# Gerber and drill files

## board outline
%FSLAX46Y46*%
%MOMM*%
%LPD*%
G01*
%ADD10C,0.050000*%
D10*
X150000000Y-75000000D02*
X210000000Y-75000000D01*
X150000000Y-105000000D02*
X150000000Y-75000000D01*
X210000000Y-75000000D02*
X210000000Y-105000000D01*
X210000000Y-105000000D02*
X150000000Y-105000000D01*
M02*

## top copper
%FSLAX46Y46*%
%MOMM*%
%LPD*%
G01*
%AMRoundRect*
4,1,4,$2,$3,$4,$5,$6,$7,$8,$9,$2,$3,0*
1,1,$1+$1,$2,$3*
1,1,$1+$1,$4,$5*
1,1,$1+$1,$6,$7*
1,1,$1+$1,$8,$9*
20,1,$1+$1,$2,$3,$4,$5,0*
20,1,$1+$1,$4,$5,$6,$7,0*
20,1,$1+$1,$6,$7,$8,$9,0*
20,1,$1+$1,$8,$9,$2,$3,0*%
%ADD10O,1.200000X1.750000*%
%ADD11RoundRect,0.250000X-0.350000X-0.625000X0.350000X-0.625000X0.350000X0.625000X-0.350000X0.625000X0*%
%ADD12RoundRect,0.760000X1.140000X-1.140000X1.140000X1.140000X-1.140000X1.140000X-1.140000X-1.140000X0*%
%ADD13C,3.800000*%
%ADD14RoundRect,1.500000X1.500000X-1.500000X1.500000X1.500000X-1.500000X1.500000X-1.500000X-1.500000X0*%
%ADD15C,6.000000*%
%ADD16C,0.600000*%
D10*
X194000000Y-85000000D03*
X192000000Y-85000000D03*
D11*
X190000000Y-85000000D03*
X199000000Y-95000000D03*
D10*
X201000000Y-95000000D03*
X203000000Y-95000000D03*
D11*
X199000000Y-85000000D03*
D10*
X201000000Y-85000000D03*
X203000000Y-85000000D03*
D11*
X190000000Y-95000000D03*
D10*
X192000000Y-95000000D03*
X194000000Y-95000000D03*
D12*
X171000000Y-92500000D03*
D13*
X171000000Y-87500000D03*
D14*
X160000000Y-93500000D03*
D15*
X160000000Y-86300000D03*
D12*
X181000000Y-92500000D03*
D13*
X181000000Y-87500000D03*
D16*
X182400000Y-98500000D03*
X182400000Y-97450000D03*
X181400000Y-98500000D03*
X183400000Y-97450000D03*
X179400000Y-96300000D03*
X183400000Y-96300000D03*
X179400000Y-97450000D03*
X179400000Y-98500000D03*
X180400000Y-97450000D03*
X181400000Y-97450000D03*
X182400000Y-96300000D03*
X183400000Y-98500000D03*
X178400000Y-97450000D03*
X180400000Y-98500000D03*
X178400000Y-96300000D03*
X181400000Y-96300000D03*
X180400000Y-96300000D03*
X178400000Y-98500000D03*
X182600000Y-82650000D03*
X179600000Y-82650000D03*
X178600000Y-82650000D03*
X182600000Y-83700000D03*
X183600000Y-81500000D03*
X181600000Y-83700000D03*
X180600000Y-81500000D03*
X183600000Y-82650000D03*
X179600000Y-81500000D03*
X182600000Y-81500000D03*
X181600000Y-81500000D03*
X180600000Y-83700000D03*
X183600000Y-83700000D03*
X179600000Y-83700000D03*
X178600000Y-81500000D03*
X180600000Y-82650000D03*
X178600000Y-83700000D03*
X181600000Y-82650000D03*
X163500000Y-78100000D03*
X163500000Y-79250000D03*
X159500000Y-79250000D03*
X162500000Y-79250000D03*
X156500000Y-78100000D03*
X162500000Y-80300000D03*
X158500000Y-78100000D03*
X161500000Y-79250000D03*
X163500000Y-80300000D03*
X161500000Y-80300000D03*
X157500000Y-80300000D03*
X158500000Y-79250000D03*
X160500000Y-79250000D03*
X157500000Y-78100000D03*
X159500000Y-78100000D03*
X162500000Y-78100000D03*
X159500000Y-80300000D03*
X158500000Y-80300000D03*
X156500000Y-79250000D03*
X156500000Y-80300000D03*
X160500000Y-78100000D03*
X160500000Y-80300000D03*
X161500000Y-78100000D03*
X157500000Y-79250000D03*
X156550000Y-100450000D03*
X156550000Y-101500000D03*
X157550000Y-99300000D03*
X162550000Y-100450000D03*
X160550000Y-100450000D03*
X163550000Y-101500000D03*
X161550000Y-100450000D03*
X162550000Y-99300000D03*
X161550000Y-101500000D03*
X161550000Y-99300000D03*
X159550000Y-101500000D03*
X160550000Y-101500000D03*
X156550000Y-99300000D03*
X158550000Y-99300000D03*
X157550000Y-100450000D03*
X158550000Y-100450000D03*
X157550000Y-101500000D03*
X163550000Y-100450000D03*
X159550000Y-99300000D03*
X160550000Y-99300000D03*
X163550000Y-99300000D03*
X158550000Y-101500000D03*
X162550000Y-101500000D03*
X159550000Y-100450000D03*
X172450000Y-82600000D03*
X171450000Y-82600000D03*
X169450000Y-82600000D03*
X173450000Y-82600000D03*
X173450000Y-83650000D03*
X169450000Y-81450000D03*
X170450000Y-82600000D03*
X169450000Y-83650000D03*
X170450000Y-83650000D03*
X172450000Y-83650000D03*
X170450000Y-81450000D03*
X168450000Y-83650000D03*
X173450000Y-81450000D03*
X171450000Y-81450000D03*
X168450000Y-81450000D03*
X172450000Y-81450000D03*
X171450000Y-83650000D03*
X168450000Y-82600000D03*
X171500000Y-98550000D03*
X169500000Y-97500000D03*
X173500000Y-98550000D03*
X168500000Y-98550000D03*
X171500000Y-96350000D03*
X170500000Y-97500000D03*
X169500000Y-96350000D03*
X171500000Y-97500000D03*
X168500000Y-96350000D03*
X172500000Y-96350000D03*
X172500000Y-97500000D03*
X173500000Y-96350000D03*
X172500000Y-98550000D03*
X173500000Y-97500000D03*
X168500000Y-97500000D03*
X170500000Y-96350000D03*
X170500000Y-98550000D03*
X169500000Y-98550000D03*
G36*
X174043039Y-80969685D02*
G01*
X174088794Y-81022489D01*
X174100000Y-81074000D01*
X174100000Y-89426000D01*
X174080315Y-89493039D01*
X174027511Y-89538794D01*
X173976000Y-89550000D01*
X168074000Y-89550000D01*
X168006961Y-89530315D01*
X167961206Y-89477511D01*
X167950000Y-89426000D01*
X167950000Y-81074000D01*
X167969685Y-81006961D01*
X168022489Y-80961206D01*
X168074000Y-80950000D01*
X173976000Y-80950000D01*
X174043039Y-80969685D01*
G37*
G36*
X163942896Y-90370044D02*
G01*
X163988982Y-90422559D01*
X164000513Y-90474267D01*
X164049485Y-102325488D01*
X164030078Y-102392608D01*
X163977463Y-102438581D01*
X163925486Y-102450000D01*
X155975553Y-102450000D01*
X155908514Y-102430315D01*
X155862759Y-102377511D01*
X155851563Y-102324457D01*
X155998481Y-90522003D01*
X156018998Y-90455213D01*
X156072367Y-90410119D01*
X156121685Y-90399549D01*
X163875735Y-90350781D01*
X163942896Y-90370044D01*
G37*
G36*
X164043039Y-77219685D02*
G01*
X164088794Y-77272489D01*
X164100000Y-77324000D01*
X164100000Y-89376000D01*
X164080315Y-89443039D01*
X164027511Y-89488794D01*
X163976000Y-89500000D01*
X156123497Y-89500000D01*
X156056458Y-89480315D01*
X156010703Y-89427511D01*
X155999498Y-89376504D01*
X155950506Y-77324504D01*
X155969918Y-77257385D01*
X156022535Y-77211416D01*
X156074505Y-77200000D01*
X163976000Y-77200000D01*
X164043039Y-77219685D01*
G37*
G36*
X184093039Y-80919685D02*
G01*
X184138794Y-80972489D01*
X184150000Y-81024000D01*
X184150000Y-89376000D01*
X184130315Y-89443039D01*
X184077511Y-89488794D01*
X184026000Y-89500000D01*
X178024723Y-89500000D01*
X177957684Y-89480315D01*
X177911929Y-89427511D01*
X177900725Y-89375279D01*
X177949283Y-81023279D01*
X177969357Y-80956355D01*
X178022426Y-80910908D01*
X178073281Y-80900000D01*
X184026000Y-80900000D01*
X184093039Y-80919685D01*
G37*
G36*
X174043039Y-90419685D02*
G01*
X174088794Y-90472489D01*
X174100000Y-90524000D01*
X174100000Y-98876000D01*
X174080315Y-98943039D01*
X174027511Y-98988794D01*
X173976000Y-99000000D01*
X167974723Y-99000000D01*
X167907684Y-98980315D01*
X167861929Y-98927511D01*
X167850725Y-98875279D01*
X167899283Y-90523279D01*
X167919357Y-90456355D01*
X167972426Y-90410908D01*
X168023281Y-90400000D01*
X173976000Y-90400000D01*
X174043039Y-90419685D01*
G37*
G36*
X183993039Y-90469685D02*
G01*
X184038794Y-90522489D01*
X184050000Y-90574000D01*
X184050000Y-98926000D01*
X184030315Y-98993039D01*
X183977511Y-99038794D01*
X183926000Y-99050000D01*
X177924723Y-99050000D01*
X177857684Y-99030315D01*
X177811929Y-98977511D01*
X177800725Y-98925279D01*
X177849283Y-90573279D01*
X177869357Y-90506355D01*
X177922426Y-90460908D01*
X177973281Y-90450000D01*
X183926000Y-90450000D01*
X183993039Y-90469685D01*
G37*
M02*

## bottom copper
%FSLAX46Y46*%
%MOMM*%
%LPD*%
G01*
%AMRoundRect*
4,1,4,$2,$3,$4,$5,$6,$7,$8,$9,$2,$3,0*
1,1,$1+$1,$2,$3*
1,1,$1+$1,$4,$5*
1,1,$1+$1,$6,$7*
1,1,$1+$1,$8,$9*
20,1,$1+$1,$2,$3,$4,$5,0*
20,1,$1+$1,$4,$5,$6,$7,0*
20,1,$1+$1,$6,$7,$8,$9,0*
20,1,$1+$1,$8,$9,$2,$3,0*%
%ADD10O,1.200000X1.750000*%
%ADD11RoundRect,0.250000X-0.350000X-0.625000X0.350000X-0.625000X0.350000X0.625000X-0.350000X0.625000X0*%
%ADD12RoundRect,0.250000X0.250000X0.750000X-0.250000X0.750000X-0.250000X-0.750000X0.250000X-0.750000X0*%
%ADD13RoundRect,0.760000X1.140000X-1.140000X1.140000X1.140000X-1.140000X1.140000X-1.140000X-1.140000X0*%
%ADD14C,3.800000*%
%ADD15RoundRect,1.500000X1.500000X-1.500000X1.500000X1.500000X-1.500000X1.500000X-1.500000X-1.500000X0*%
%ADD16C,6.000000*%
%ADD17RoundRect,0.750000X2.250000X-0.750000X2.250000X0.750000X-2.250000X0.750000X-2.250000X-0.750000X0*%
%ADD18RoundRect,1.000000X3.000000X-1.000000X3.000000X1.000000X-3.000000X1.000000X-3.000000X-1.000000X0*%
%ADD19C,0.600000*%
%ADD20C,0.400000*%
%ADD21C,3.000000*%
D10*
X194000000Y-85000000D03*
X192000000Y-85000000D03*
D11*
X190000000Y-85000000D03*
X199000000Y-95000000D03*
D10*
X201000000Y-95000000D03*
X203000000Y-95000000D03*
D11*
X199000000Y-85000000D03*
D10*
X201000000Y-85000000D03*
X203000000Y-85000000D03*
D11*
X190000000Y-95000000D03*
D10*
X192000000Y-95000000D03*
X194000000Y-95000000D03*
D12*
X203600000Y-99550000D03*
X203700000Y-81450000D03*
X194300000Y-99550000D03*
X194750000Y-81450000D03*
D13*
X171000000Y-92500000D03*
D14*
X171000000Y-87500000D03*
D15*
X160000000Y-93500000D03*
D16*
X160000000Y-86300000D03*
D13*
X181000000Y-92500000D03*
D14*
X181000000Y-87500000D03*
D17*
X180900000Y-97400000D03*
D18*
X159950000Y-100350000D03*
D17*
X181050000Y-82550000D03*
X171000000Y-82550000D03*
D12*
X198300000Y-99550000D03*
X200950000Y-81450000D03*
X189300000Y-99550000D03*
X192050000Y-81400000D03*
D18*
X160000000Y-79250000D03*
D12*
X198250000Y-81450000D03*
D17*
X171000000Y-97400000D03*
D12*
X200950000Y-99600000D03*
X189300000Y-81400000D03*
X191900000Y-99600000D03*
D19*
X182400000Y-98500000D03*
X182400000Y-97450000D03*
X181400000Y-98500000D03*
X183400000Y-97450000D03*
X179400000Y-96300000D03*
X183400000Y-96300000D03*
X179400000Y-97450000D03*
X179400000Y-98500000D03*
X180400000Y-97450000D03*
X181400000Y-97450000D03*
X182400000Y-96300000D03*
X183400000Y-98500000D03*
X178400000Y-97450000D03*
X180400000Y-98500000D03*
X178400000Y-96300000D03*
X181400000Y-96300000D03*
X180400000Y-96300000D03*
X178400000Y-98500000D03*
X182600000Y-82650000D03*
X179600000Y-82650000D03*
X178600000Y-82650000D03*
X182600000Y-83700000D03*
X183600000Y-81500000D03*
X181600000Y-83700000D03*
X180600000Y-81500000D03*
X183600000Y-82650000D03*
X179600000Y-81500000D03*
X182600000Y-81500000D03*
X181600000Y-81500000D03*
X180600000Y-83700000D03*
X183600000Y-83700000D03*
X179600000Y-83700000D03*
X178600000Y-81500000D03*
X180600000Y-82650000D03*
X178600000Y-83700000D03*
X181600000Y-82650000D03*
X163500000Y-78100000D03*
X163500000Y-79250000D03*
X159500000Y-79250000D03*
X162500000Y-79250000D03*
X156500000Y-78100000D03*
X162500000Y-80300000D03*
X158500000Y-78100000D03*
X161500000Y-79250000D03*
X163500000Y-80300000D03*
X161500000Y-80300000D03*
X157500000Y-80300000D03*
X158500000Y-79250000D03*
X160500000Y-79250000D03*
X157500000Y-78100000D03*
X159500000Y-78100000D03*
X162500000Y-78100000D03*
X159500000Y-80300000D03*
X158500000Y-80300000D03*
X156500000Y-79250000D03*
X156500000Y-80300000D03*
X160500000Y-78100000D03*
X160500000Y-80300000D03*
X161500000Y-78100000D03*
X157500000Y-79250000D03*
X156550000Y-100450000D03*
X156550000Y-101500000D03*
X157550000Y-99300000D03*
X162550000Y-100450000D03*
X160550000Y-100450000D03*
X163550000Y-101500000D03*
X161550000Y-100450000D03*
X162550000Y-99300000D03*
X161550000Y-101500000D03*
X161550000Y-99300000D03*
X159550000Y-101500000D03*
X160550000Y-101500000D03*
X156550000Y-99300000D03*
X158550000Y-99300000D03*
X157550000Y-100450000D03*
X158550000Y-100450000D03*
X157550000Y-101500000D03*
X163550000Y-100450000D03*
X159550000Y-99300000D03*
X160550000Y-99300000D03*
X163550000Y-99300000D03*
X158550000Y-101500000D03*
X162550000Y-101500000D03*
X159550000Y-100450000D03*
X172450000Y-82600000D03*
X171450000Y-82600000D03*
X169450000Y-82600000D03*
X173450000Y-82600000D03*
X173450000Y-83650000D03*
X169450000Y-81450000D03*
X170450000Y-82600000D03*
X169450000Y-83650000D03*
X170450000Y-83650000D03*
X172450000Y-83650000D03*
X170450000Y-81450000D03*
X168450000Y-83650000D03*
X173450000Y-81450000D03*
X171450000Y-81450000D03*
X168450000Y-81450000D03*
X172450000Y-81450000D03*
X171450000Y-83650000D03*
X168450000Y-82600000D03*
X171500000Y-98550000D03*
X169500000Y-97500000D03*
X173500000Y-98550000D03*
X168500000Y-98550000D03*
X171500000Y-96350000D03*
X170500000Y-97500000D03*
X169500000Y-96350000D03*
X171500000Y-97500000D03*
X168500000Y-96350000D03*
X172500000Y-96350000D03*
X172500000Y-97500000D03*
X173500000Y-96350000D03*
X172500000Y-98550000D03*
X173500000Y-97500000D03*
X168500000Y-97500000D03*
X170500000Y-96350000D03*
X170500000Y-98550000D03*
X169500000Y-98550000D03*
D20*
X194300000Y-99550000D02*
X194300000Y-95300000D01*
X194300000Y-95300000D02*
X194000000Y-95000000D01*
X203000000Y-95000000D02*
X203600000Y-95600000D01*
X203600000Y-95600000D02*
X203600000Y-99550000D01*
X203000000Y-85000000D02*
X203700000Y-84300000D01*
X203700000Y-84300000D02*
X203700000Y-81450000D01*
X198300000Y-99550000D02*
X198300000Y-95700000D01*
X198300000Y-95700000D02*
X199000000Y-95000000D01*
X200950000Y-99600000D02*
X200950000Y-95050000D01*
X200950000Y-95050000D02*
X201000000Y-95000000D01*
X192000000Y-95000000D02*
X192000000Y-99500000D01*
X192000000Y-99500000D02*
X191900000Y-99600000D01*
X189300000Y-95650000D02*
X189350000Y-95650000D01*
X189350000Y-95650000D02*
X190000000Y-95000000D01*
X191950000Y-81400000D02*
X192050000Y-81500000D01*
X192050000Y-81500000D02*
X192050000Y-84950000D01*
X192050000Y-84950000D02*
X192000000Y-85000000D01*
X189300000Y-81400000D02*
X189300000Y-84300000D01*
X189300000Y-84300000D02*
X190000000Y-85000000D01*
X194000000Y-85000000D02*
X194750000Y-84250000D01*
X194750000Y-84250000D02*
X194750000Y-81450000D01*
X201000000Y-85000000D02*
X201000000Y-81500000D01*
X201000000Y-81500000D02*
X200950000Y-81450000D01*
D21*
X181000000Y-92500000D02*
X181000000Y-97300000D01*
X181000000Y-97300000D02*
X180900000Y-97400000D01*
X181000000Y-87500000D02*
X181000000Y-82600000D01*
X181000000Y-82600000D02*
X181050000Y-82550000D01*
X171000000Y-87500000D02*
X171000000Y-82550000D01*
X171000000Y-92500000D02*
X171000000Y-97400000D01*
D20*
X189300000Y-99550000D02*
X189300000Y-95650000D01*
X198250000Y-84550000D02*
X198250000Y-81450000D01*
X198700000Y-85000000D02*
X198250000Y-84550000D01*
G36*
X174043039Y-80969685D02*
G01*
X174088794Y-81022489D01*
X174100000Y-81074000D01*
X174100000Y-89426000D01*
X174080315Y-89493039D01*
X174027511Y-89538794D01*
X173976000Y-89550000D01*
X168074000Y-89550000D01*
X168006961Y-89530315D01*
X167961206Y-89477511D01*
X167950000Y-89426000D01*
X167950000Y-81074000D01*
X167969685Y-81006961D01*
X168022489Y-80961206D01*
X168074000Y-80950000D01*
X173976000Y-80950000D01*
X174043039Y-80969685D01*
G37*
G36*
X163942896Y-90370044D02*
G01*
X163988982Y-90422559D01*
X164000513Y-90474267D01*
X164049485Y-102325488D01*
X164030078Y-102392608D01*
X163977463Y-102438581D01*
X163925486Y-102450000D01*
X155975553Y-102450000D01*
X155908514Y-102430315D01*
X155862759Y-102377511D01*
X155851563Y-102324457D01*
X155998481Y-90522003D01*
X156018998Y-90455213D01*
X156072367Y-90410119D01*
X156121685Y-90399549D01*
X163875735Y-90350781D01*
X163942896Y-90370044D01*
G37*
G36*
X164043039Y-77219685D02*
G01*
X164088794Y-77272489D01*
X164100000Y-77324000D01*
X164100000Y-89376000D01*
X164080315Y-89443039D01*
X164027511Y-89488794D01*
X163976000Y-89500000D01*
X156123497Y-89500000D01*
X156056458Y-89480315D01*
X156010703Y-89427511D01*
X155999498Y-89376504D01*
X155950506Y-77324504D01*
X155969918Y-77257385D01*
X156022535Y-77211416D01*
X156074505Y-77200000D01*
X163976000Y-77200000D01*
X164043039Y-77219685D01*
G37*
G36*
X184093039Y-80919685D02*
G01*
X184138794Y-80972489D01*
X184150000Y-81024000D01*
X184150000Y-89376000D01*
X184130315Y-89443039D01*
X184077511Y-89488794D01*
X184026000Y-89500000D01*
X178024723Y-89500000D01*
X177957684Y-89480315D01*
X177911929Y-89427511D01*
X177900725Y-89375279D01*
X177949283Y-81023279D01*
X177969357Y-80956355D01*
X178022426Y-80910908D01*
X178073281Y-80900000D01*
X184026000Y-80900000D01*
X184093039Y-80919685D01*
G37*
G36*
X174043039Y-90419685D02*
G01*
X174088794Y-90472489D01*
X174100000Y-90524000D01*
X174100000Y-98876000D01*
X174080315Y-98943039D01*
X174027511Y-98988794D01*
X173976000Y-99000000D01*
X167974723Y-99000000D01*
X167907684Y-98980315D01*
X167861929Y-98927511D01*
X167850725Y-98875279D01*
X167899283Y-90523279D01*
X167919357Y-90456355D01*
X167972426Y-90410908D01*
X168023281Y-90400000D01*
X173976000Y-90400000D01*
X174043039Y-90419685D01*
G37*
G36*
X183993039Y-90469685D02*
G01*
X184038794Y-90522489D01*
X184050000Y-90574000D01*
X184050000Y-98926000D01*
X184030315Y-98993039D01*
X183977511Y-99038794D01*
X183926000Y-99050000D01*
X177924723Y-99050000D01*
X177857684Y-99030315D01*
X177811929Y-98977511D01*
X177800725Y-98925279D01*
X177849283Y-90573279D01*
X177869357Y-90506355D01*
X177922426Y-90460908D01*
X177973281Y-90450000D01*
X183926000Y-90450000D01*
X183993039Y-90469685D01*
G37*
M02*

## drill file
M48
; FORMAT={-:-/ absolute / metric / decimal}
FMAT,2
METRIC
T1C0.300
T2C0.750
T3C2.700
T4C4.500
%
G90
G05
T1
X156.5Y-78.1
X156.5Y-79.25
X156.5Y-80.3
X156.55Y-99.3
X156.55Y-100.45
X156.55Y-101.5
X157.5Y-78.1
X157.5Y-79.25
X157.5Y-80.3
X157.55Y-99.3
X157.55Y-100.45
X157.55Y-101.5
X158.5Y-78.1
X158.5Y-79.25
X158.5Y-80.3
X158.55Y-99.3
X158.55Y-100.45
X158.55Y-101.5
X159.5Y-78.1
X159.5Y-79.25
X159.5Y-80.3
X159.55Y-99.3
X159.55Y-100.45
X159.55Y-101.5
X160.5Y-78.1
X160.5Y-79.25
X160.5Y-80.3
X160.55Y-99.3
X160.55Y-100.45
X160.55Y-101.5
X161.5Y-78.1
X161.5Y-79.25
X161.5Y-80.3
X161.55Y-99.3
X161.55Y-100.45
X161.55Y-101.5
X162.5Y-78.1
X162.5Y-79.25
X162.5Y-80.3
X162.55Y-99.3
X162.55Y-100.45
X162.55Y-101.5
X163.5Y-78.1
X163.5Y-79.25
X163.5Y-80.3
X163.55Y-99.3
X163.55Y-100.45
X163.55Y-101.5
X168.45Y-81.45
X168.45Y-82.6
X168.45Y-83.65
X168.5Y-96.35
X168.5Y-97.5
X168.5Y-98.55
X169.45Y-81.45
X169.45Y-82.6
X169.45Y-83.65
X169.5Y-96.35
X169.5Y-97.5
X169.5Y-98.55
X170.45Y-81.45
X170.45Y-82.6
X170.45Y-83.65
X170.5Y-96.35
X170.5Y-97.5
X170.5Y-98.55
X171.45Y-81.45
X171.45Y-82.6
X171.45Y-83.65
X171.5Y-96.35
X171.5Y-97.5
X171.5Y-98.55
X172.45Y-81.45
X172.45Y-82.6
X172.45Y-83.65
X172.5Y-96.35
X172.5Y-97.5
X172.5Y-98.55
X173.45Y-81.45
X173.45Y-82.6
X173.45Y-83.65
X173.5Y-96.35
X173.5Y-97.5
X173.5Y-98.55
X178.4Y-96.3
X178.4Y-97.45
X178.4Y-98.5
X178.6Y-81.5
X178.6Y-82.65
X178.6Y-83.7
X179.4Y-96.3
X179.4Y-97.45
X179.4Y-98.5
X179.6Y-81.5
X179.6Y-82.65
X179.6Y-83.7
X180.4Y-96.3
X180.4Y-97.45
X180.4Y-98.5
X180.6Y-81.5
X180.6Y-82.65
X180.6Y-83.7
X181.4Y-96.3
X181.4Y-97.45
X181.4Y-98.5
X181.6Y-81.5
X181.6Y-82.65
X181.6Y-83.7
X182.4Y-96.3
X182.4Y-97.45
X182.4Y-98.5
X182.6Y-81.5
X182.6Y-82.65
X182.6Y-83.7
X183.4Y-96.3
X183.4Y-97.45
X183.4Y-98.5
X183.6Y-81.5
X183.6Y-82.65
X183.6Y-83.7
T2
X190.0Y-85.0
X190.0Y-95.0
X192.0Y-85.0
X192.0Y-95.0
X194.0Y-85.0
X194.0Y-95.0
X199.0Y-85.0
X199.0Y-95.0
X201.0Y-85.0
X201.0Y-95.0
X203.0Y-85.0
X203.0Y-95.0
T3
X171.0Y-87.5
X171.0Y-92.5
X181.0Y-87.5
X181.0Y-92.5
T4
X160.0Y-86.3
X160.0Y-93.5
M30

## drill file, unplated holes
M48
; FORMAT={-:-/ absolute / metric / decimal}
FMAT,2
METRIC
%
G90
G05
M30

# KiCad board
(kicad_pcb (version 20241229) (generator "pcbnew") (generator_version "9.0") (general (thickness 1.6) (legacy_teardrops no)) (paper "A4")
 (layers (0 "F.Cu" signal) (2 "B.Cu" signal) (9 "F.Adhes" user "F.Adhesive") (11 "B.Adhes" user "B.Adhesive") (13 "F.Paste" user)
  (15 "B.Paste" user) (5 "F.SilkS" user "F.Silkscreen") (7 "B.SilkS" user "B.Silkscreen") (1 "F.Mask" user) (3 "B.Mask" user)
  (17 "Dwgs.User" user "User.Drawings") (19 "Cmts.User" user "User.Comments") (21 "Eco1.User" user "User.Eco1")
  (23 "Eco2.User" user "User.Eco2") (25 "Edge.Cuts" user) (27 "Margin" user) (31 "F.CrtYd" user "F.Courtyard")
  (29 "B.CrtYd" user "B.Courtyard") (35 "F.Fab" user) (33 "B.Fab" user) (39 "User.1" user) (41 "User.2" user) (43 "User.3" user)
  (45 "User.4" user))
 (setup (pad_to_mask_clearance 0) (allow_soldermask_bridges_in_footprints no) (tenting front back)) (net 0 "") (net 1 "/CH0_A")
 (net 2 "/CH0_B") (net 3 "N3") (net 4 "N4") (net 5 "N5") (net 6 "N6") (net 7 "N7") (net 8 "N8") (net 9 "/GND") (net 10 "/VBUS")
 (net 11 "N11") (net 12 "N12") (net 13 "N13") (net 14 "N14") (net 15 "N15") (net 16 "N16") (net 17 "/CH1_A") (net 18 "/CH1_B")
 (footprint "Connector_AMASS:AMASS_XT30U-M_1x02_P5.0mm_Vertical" (layer "F.Cu") (at 171 92.5 90)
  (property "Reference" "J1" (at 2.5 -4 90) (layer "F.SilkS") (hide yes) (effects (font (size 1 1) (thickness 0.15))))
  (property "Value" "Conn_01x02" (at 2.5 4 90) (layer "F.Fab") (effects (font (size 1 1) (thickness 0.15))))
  (pad "1" thru_hole roundrect (at 0 0 90) (size 3.8 3.8) (drill 2.7) (layers "*.Cu" "*.Mask") (remove_unused_layers no)
   (roundrect_rratio 0.2) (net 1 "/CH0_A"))
  (pad "2" thru_hole circle (at 5 0 90) (size 3.8 3.8) (drill 2.7) (layers "*.Cu" "*.Mask") (remove_unused_layers no) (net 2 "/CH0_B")))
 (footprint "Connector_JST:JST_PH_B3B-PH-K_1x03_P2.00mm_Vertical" (layer "F.Cu") (at 190 85)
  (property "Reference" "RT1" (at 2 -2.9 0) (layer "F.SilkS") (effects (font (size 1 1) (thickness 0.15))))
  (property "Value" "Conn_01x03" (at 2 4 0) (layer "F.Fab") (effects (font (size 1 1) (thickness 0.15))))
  (pad "1" thru_hole roundrect (at 0 0) (size 1.2 1.75) (drill 0.75) (layers "*.Cu" "*.Mask") (remove_unused_layers no)
   (roundrect_rratio 0.208333) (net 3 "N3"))
  (pad "2" thru_hole oval (at 2 0) (size 1.2 1.75) (drill 0.75) (layers "*.Cu" "*.Mask") (remove_unused_layers no) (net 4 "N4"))
  (pad "3" thru_hole oval (at 4 0) (size 1.2 1.75) (drill 0.75) (layers "*.Cu" "*.Mask") (remove_unused_layers no) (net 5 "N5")))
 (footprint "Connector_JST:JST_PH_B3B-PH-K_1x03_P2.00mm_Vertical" (layer "F.Cu") (at 199 95)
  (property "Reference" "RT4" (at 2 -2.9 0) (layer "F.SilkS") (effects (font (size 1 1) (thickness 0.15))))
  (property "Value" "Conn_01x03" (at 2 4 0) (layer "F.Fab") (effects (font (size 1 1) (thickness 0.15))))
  (pad "1" thru_hole roundrect (at 0 0) (size 1.2 1.75) (drill 0.75) (layers "*.Cu" "*.Mask") (remove_unused_layers no)
   (roundrect_rratio 0.208333) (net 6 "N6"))
  (pad "2" thru_hole oval (at 2 0) (size 1.2 1.75) (drill 0.75) (layers "*.Cu" "*.Mask") (remove_unused_layers no) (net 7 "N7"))
  (pad "3" thru_hole oval (at 4 0) (size 1.2 1.75) (drill 0.75) (layers "*.Cu" "*.Mask") (remove_unused_layers no) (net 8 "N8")))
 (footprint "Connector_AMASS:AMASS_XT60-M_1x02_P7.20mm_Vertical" (layer "F.Cu") (at 160 93.5 90)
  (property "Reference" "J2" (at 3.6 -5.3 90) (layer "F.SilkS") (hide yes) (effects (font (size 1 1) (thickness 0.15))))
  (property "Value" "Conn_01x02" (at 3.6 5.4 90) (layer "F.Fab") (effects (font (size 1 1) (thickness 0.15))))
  (pad "1" thru_hole roundrect (at 0 0 90) (size 6 6) (drill 4.5) (layers "*.Cu" "*.Mask") (remove_unused_layers no) (roundrect_rratio 0.25)
   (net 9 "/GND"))
  (pad "2" thru_hole circle (at 7.2 0 90) (size 6 6) (drill 4.5) (layers "*.Cu" "*.Mask") (remove_unused_layers no) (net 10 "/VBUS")))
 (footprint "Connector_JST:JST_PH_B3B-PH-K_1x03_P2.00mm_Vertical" (layer "F.Cu") (at 199 85)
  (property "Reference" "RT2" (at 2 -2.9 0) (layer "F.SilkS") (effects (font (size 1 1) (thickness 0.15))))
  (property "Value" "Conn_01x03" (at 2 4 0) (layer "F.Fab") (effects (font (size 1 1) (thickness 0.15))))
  (pad "1" thru_hole roundrect (at 0 0) (size 1.2 1.75) (drill 0.75) (layers "*.Cu" "*.Mask") (remove_unused_layers no)
   (roundrect_rratio 0.208333) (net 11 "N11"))
  (pad "2" thru_hole oval (at 2 0) (size 1.2 1.75) (drill 0.75) (layers "*.Cu" "*.Mask") (remove_unused_layers no) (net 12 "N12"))
  (pad "3" thru_hole oval (at 4 0) (size 1.2 1.75) (drill 0.75) (layers "*.Cu" "*.Mask") (remove_unused_layers no) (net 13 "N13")))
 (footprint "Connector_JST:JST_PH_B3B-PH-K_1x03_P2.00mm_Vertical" (layer "F.Cu") (at 190 95)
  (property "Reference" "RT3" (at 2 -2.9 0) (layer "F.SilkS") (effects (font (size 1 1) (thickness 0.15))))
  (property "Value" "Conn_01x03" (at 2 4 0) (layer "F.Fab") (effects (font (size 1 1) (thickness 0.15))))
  (pad "1" thru_hole roundrect (at 0 0) (size 1.2 1.75) (drill 0.75) (layers "*.Cu" "*.Mask") (remove_unused_layers no)
   (roundrect_rratio 0.208333) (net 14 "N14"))
  (pad "2" thru_hole oval (at 2 0) (size 1.2 1.75) (drill 0.75) (layers "*.Cu" "*.Mask") (remove_unused_layers no) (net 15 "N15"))
  (pad "3" thru_hole oval (at 4 0) (size 1.2 1.75) (drill 0.75) (layers "*.Cu" "*.Mask") (remove_unused_layers no) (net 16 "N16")))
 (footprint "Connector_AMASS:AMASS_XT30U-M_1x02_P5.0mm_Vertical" (layer "F.Cu") (at 181 92.5 90)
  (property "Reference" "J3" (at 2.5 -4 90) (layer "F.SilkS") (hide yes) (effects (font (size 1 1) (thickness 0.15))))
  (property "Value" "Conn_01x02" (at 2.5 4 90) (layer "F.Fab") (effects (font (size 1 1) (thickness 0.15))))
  (pad "1" thru_hole roundrect (at 0 0 90) (size 3.8 3.8) (drill 2.7) (layers "*.Cu" "*.Mask") (remove_unused_layers no)
   (roundrect_rratio 0.2) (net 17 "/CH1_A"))
  (pad "2" thru_hole circle (at 5 0 90) (size 3.8 3.8) (drill 2.7) (layers "*.Cu" "*.Mask") (remove_unused_layers no) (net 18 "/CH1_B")))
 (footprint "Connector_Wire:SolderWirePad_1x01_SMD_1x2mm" (layer "B.Cu") (at 203.7 81.45 180)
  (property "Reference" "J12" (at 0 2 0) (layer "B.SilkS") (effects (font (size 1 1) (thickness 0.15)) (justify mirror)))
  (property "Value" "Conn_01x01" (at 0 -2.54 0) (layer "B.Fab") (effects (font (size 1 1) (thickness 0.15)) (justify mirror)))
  (pad "1" smd roundrect (at 0 0 180) (size 1 2) (layers "B.Cu" "B.Mask") (roundrect_rratio 0.25) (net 13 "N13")))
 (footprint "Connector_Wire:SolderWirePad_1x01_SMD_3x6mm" (layer "B.Cu") (at 180.9 97.4 90)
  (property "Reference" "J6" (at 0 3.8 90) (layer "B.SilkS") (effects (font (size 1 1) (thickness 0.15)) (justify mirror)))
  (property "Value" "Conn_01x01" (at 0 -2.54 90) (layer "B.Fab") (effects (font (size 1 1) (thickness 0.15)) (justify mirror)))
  (pad "1" smd roundrect (at 0 0 90) (size 3 6) (layers "B.Cu" "B.Mask") (roundrect_rratio 0.25) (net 17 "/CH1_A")))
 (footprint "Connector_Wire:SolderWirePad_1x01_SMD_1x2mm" (layer "B.Cu") (at 203.6 99.55 180)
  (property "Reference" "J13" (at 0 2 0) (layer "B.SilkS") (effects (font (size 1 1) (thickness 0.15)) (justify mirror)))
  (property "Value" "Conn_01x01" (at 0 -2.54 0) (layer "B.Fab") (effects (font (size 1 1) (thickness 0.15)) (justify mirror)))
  (pad "1" smd roundrect (at 0 0 180) (size 1 2) (layers "B.Cu" "B.Mask") (roundrect_rratio 0.25) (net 8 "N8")))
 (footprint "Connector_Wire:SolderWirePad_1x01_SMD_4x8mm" (layer "B.Cu") (at 159.95 100.35 90)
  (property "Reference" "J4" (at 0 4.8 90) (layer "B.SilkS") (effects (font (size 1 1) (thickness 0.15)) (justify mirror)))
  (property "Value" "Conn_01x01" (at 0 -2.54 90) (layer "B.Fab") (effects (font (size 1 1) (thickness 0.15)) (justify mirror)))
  (pad "1" smd roundrect (at 0 0 90) (size 4 8) (layers "B.Cu" "B.Mask") (roundrect_rratio 0.25) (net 9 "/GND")))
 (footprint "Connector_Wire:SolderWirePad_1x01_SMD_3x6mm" (layer "B.Cu") (at 181.05 82.55 90)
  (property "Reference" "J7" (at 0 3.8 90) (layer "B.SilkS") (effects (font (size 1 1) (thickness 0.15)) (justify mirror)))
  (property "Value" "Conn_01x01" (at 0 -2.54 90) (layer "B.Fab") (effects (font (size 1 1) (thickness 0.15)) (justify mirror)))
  (pad "1" smd roundrect (at 0 0 90) (size 3 6) (layers "B.Cu" "B.Mask") (roundrect_rratio 0.25) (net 18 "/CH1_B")))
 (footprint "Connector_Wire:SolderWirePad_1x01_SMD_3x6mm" (layer "B.Cu") (at 171 82.55 90)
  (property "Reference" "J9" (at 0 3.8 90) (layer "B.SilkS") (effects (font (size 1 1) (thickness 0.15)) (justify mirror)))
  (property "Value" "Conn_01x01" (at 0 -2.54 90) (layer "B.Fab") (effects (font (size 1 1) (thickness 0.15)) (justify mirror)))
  (pad "1" smd roundrect (at 0 0 90) (size 3 6) (layers "B.Cu" "B.Mask") (roundrect_rratio 0.25) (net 2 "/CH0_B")))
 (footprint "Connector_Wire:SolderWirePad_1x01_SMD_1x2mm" (layer "B.Cu") (at 198.3 99.55 180)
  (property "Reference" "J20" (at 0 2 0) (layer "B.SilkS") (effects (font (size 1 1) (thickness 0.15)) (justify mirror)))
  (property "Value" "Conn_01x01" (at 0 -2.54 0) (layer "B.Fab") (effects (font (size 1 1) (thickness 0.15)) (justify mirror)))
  (pad "1" smd roundrect (at 0 0 180) (size 1 2) (layers "B.Cu" "B.Mask") (roundrect_rratio 0.25) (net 6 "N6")))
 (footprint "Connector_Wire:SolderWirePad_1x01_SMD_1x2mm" (layer "B.Cu") (at 200.95 81.45 180)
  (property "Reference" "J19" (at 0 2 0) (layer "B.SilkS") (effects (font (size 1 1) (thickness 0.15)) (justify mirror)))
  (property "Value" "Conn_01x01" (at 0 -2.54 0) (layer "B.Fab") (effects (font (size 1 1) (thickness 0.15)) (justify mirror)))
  (pad "1" smd roundrect (at 0 0 180) (size 1 2) (layers "B.Cu" "B.Mask") (roundrect_rratio 0.25) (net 12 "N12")))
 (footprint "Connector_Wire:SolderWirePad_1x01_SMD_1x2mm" (layer "B.Cu") (at 189.3 99.55 180)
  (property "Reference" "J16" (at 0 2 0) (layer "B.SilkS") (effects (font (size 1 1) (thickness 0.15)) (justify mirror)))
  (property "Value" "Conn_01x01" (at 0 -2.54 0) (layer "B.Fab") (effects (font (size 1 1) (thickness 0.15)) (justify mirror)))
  (pad "1" smd roundrect (at 0 0 180) (size 1 2) (layers "B.Cu" "B.Mask") (roundrect_rratio 0.25) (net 14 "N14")))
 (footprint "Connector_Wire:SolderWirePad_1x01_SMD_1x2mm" (layer "B.Cu") (at 192.05 81.4 180)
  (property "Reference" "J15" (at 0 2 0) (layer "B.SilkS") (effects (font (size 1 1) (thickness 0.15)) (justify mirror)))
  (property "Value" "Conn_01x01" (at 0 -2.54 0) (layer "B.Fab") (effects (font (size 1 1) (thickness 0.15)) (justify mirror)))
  (pad "1" smd roundrect (at 0 0 180) (size 1 2) (layers "B.Cu" "B.Mask") (roundrect_rratio 0.25) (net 4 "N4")))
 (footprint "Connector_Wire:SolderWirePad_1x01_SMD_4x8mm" (layer "B.Cu") (at 160 79.25 90)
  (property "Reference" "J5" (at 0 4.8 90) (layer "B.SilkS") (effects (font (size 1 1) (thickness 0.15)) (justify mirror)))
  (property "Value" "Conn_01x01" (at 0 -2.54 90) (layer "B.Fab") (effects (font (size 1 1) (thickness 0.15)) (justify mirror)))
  (pad "1" smd roundrect (at 0 0 90) (size 4 8) (layers "B.Cu" "B.Mask") (roundrect_rratio 0.25) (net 10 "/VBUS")))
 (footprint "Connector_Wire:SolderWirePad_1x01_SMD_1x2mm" (layer "B.Cu") (at 194.75 81.45 180)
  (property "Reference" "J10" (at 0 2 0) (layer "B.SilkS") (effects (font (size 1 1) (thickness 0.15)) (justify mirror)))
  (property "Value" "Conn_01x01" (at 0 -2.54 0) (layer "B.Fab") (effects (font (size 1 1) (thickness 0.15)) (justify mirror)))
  (pad "1" smd roundrect (at 0 0 180) (size 1 2) (layers "B.Cu" "B.Mask") (roundrect_rratio 0.25) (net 5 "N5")))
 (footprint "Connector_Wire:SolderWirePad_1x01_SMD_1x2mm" (layer "B.Cu") (at 194.3 99.55 180)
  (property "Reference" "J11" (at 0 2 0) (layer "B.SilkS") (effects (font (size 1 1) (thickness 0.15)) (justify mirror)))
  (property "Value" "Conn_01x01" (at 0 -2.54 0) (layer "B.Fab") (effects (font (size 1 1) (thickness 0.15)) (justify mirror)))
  (pad "1" smd roundrect (at 0 0 180) (size 1 2) (layers "B.Cu" "B.Mask") (roundrect_rratio 0.25) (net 16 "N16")))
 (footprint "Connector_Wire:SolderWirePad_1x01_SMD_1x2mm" (layer "B.Cu") (at 198.25 81.45 180)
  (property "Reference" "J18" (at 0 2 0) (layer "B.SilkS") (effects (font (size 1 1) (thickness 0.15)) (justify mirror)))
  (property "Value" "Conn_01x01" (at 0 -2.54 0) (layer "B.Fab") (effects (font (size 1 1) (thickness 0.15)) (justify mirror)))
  (pad "1" smd roundrect (at 0 0 180) (size 1 2) (layers "B.Cu" "B.Mask") (roundrect_rratio 0.25) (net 11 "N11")))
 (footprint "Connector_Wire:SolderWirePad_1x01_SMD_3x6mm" (layer "B.Cu") (at 171 97.4 90)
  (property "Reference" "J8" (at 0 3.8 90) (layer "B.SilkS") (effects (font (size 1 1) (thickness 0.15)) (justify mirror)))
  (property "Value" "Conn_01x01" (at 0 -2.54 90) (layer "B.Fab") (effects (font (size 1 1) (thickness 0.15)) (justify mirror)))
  (pad "1" smd roundrect (at 0 0 90) (size 3 6) (layers "B.Cu" "B.Mask") (roundrect_rratio 0.25) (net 1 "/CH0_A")))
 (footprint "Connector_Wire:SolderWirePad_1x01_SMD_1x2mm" (layer "B.Cu") (at 200.95 99.6 180)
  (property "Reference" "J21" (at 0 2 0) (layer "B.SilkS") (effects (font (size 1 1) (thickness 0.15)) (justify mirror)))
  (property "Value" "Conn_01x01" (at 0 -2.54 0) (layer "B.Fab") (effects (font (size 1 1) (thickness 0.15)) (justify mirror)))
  (pad "1" smd roundrect (at 0 0 180) (size 1 2) (layers "B.Cu" "B.Mask") (roundrect_rratio 0.25) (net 7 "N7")))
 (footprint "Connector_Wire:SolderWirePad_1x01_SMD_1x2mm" (layer "B.Cu") (at 189.3 81.4 180)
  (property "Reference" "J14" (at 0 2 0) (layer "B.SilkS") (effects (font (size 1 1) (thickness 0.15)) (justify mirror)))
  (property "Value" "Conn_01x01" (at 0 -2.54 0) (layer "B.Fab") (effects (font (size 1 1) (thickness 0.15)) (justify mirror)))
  (pad "1" smd roundrect (at 0 0 180) (size 1 2) (layers "B.Cu" "B.Mask") (roundrect_rratio 0.25) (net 3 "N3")))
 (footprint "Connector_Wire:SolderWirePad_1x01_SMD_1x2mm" (layer "B.Cu") (at 191.9 99.6 180)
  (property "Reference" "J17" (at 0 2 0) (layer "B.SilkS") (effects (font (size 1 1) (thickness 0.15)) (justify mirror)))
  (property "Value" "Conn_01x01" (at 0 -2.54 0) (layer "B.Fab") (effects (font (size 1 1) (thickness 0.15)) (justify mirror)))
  (pad "1" smd roundrect (at 0 0 180) (size 1 2) (layers "B.Cu" "B.Mask") (roundrect_rratio 0.25) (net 15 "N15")))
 (gr_line (start 150 75) (end 210 75) (stroke (width 0.05) (type solid)) (layer "Edge.Cuts"))
 (gr_line (start 150 105) (end 150 75) (stroke (width 0.05) (type solid)) (layer "Edge.Cuts"))
 (gr_line (start 210 75) (end 210 105) (stroke (width 0.05) (type solid)) (layer "Edge.Cuts"))
 (gr_line (start 210 105) (end 150 105) (stroke (width 0.05) (type solid)) (layer "Edge.Cuts"))
 (via (at 182.4 98.5) (size 0.6) (drill 0.3) (layers "F.Cu" "B.Cu") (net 17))
 (via (at 182.4 97.45) (size 0.6) (drill 0.3) (layers "F.Cu" "B.Cu") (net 17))
 (via (at 181.4 98.5) (size 0.6) (drill 0.3) (layers "F.Cu" "B.Cu") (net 17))
 (via (at 183.4 97.45) (size 0.6) (drill 0.3) (layers "F.Cu" "B.Cu") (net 17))
 (via (at 179.4 96.3) (size 0.6) (drill 0.3) (layers "F.Cu" "B.Cu") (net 17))
 (via (at 183.4 96.3) (size 0.6) (drill 0.3) (layers "F.Cu" "B.Cu") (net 17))
 (via (at 179.4 97.45) (size 0.6) (drill 0.3) (layers "F.Cu" "B.Cu") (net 17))
 (via (at 179.4 98.5) (size 0.6) (drill 0.3) (layers "F.Cu" "B.Cu") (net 17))
 (via (at 180.4 97.45) (size 0.6) (drill 0.3) (layers "F.Cu" "B.Cu") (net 17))
 (via (at 181.4 97.45) (size 0.6) (drill 0.3) (layers "F.Cu" "B.Cu") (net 17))
 (via (at 182.4 96.3) (size 0.6) (drill 0.3) (layers "F.Cu" "B.Cu") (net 17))
 (via (at 183.4 98.5) (size 0.6) (drill 0.3) (layers "F.Cu" "B.Cu") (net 17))
 (via (at 178.4 97.45) (size 0.6) (drill 0.3) (layers "F.Cu" "B.Cu") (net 17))
 (via (at 180.4 98.5) (size 0.6) (drill 0.3) (layers "F.Cu" "B.Cu") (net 17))
 (via (at 178.4 96.3) (size 0.6) (drill 0.3) (layers "F.Cu" "B.Cu") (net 17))
 (via (at 181.4 96.3) (size 0.6) (drill 0.3) (layers "F.Cu" "B.Cu") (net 17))
 (via (at 180.4 96.3) (size 0.6) (drill 0.3) (layers "F.Cu" "B.Cu") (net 17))
 (via (at 178.4 98.5) (size 0.6) (drill 0.3) (layers "F.Cu" "B.Cu") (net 17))
 (segment (start 181 92.5) (end 181 97.3) (width 3) (layer "B.Cu") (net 17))
 (segment (start 181 97.3) (end 180.9 97.4) (width 3) (layer "B.Cu") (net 17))
 (via (at 182.6 82.65) (size 0.6) (drill 0.3) (layers "F.Cu" "B.Cu") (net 18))
 (via (at 179.6 82.65) (size 0.6) (drill 0.3) (layers "F.Cu" "B.Cu") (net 18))
 (via (at 178.6 82.65) (size 0.6) (drill 0.3) (layers "F.Cu" "B.Cu") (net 18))
 (via (at 182.6 83.7) (size 0.6) (drill 0.3) (layers "F.Cu" "B.Cu") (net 18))
 (via (at 183.6 81.5) (size 0.6) (drill 0.3) (layers "F.Cu" "B.Cu") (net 18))
 (via (at 181.6 83.7) (size 0.6) (drill 0.3) (layers "F.Cu" "B.Cu") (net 18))
 (via (at 180.6 81.5) (size 0.6) (drill 0.3) (layers "F.Cu" "B.Cu") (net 18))
 (via (at 183.6 82.65) (size 0.6) (drill 0.3) (layers "F.Cu" "B.Cu") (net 18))
 (via (at 179.6 81.5) (size 0.6) (drill 0.3) (layers "F.Cu" "B.Cu") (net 18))
 (via (at 182.6 81.5) (size 0.6) (drill 0.3) (layers "F.Cu" "B.Cu") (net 18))
 (via (at 181.6 81.5) (size 0.6) (drill 0.3) (layers "F.Cu" "B.Cu") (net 18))
 (via (at 180.6 83.7) (size 0.6) (drill 0.3) (layers "F.Cu" "B.Cu") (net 18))
 (via (at 183.6 83.7) (size 0.6) (drill 0.3) (layers "F.Cu" "B.Cu") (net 18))
 (via (at 179.6 83.7) (size 0.6) (drill 0.3) (layers "F.Cu" "B.Cu") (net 18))
 (via (at 178.6 81.5) (size 0.6) (drill 0.3) (layers "F.Cu" "B.Cu") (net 18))
 (via (at 180.6 82.65) (size 0.6) (drill 0.3) (layers "F.Cu" "B.Cu") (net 18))
 (via (at 178.6 83.7) (size 0.6) (drill 0.3) (layers "F.Cu" "B.Cu") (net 18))
 (via (at 181.6 82.65) (size 0.6) (drill 0.3) (layers "F.Cu" "B.Cu") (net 18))
 (segment (start 181 87.5) (end 181 82.6) (width 3) (layer "B.Cu") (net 18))
 (segment (start 181 82.6) (end 181.05 82.55) (width 3) (layer "B.Cu") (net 18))
 (via (at 163.5 78.1) (size 0.6) (drill 0.3) (layers "F.Cu" "B.Cu") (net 10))
 (via (at 163.5 79.25) (size 0.6) (drill 0.3) (layers "F.Cu" "B.Cu") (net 10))
 (via (at 159.5 79.25) (size 0.6) (drill 0.3) (layers "F.Cu" "B.Cu") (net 10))
 (via (at 162.5 79.25) (size 0.6) (drill 0.3) (layers "F.Cu" "B.Cu") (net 10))
 (via (at 156.5 78.1) (size 0.6) (drill 0.3) (layers "F.Cu" "B.Cu") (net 10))
 (via (at 162.5 80.3) (size 0.6) (drill 0.3) (layers "F.Cu" "B.Cu") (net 10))
 (via (at 158.5 78.1) (size 0.6) (drill 0.3) (layers "F.Cu" "B.Cu") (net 10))
 (via (at 161.5 79.25) (size 0.6) (drill 0.3) (layers "F.Cu" "B.Cu") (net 10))
 (via (at 163.5 80.3) (size 0.6) (drill 0.3) (layers "F.Cu" "B.Cu") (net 10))
 (via (at 161.5 80.3) (size 0.6) (drill 0.3) (layers "F.Cu" "B.Cu") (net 10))
 (via (at 157.5 80.3) (size 0.6) (drill 0.3) (layers "F.Cu" "B.Cu") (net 10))
 (via (at 158.5 79.25) (size 0.6) (drill 0.3) (layers "F.Cu" "B.Cu") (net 10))
 (via (at 160.5 79.25) (size 0.6) (drill 0.3) (layers "F.Cu" "B.Cu") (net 10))
 (via (at 157.5 78.1) (size 0.6) (drill 0.3) (layers "F.Cu" "B.Cu") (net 10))
 (via (at 159.5 78.1) (size 0.6) (drill 0.3) (layers "F.Cu" "B.Cu") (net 10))
 (via (at 162.5 78.1) (size 0.6) (drill 0.3) (layers "F.Cu" "B.Cu") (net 10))
 (via (at 159.5 80.3) (size 0.6) (drill 0.3) (layers "F.Cu" "B.Cu") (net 10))
 (via (at 158.5 80.3) (size 0.6) (drill 0.3) (layers "F.Cu" "B.Cu") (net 10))
 (via (at 156.5 79.25) (size 0.6) (drill 0.3) (layers "F.Cu" "B.Cu") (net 10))
 (via (at 156.5 80.3) (size 0.6) (drill 0.3) (layers "F.Cu" "B.Cu") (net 10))
 (via (at 160.5 78.1) (size 0.6) (drill 0.3) (layers "F.Cu" "B.Cu") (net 10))
 (via (at 160.5 80.3) (size 0.6) (drill 0.3) (layers "F.Cu" "B.Cu") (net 10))
 (via (at 161.5 78.1) (size 0.6) (drill 0.3) (layers "F.Cu" "B.Cu") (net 10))
 (via (at 157.5 79.25) (size 0.6) (drill 0.3) (layers "F.Cu" "B.Cu") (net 10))
 (via (at 156.55 100.45) (size 0.6) (drill 0.3) (layers "F.Cu" "B.Cu") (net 9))
 (via (at 156.55 101.5) (size 0.6) (drill 0.3) (layers "F.Cu" "B.Cu") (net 9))
 (via (at 157.55 99.3) (size 0.6) (drill 0.3) (layers "F.Cu" "B.Cu") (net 9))
 (via (at 162.55 100.45) (size 0.6) (drill 0.3) (layers "F.Cu" "B.Cu") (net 9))
 (via (at 160.55 100.45) (size 0.6) (drill 0.3) (layers "F.Cu" "B.Cu") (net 9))
 (via (at 163.55 101.5) (size 0.6) (drill 0.3) (layers "F.Cu" "B.Cu") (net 9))
 (via (at 161.55 100.45) (size 0.6) (drill 0.3) (layers "F.Cu" "B.Cu") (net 9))
 (via (at 162.55 99.3) (size 0.6) (drill 0.3) (layers "F.Cu" "B.Cu") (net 9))
 (via (at 161.55 101.5) (size 0.6) (drill 0.3) (layers "F.Cu" "B.Cu") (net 9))
 (via (at 161.55 99.3) (size 0.6) (drill 0.3) (layers "F.Cu" "B.Cu") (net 9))
 (via (at 159.55 101.5) (size 0.6) (drill 0.3) (layers "F.Cu" "B.Cu") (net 9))
 (via (at 160.55 101.5) (size 0.6) (drill 0.3) (layers "F.Cu" "B.Cu") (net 9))
 (via (at 156.55 99.3) (size 0.6) (drill 0.3) (layers "F.Cu" "B.Cu") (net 9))
 (via (at 158.55 99.3) (size 0.6) (drill 0.3) (layers "F.Cu" "B.Cu") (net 9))
 (via (at 157.55 100.45) (size 0.6) (drill 0.3) (layers "F.Cu" "B.Cu") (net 9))
 (via (at 158.55 100.45) (size 0.6) (drill 0.3) (layers "F.Cu" "B.Cu") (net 9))
 (via (at 157.55 101.5) (size 0.6) (drill 0.3) (layers "F.Cu" "B.Cu") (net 9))
 (via (at 163.55 100.45) (size 0.6) (drill 0.3) (layers "F.Cu" "B.Cu") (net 9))
 (via (at 159.55 99.3) (size 0.6) (drill 0.3) (layers "F.Cu" "B.Cu") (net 9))
 (via (at 160.55 99.3) (size 0.6) (drill 0.3) (layers "F.Cu" "B.Cu") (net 9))
 (via (at 163.55 99.3) (size 0.6) (drill 0.3) (layers "F.Cu" "B.Cu") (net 9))
 (via (at 158.55 101.5) (size 0.6) (drill 0.3) (layers "F.Cu" "B.Cu") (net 9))
 (via (at 162.55 101.5) (size 0.6) (drill 0.3) (layers "F.Cu" "B.Cu") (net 9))
 (via (at 159.55 100.45) (size 0.6) (drill 0.3) (layers "F.Cu" "B.Cu") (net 9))
 (via (at 172.45 82.6) (size 0.6) (drill 0.3) (layers "F.Cu" "B.Cu") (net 2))
 (via (at 171.45 82.6) (size 0.6) (drill 0.3) (layers "F.Cu" "B.Cu") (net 2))
 (via (at 169.45 82.6) (size 0.6) (drill 0.3) (layers "F.Cu" "B.Cu") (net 2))
 (via (at 173.45 82.6) (size 0.6) (drill 0.3) (layers "F.Cu" "B.Cu") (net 2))
 (via (at 173.45 83.65) (size 0.6) (drill 0.3) (layers "F.Cu" "B.Cu") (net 2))
 (via (at 169.45 81.45) (size 0.6) (drill 0.3) (layers "F.Cu" "B.Cu") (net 2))
 (via (at 170.45 82.6) (size 0.6) (drill 0.3) (layers "F.Cu" "B.Cu") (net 2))
 (via (at 169.45 83.65) (size 0.6) (drill 0.3) (layers "F.Cu" "B.Cu") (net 2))
 (via (at 170.45 83.65) (size 0.6) (drill 0.3) (layers "F.Cu" "B.Cu") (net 2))
 (via (at 172.45 83.65) (size 0.6) (drill 0.3) (layers "F.Cu" "B.Cu") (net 2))
 (via (at 170.45 81.45) (size 0.6) (drill 0.3) (layers "F.Cu" "B.Cu") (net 2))
 (via (at 168.45 83.65) (size 0.6) (drill 0.3) (layers "F.Cu" "B.Cu") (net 2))
 (via (at 173.45 81.45) (size 0.6) (drill 0.3) (layers "F.Cu" "B.Cu") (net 2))
 (via (at 171.45 81.45) (size 0.6) (drill 0.3) (layers "F.Cu" "B.Cu") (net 2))
 (via (at 168.45 81.45) (size 0.6) (drill 0.3) (layers "F.Cu" "B.Cu") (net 2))
 (via (at 172.45 81.45) (size 0.6) (drill 0.3) (layers "F.Cu" "B.Cu") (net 2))
 (via (at 171.45 83.65) (size 0.6) (drill 0.3) (layers "F.Cu" "B.Cu") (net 2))
 (via (at 168.45 82.6) (size 0.6) (drill 0.3) (layers "F.Cu" "B.Cu") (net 2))
 (segment (start 171 87.5) (end 171 82.55) (width 3) (layer "B.Cu") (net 2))
 (via (at 171.5 98.55) (size 0.6) (drill 0.3) (layers "F.Cu" "B.Cu") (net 1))
 (via (at 169.5 97.5) (size 0.6) (drill 0.3) (layers "F.Cu" "B.Cu") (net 1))
 (via (at 173.5 98.55) (size 0.6) (drill 0.3) (layers "F.Cu" "B.Cu") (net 1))
 (via (at 168.5 98.55) (size 0.6) (drill 0.3) (layers "F.Cu" "B.Cu") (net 1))
 (via (at 171.5 96.35) (size 0.6) (drill 0.3) (layers "F.Cu" "B.Cu") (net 1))
 (via (at 170.5 97.5) (size 0.6) (drill 0.3) (layers "F.Cu" "B.Cu") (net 1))
 (via (at 169.5 96.35) (size 0.6) (drill 0.3) (layers "F.Cu" "B.Cu") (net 1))
 (via (at 171.5 97.5) (size 0.6) (drill 0.3) (layers "F.Cu" "B.Cu") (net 1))
 (via (at 168.5 96.35) (size 0.6) (drill 0.3) (layers "F.Cu" "B.Cu") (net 1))
 (via (at 172.5 96.35) (size 0.6) (drill 0.3) (layers "F.Cu" "B.Cu") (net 1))
 (via (at 172.5 97.5) (size 0.6) (drill 0.3) (layers "F.Cu" "B.Cu") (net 1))
 (via (at 173.5 96.35) (size 0.6) (drill 0.3) (layers "F.Cu" "B.Cu") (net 1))
 (via (at 172.5 98.55) (size 0.6) (drill 0.3) (layers "F.Cu" "B.Cu") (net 1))
 (via (at 173.5 97.5) (size 0.6) (drill 0.3) (layers "F.Cu" "B.Cu") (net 1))
 (via (at 168.5 97.5) (size 0.6) (drill 0.3) (layers "F.Cu" "B.Cu") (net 1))
 (via (at 170.5 96.35) (size 0.6) (drill 0.3) (layers "F.Cu" "B.Cu") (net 1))
 (via (at 170.5 98.55) (size 0.6) (drill 0.3) (layers "F.Cu" "B.Cu") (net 1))
 (via (at 169.5 98.55) (size 0.6) (drill 0.3) (layers "F.Cu" "B.Cu") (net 1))
 (segment (start 171 92.5) (end 171 97.4) (width 3) (layer "B.Cu") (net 1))
 (segment (start 189.3 84.3) (end 190 85) (width 0.4) (layer "B.Cu") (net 3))
 (segment (start 189.3 81.4) (end 189.3 84.3) (width 0.4) (layer "B.Cu") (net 3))
 (segment (start 194.75 84.25) (end 194.75 81.45) (width 0.4) (layer "B.Cu") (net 5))
 (segment (start 194 85) (end 194.75 84.25) (width 0.4) (layer "B.Cu") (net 5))
 (segment (start 192.05 84.95) (end 192 85) (width 0.4) (layer "B.Cu") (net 4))
 (segment (start 191.95 81.4) (end 192.05 81.5) (width 0.4) (layer "B.Cu") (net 4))
 (segment (start 192.05 81.5) (end 192.05 84.95) (width 0.4) (layer "B.Cu") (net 4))
 (segment (start 194.3 95.3) (end 194 95) (width 0.4) (layer "B.Cu") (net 16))
 (segment (start 194.3 99.55) (end 194.3 95.3) (width 0.4) (layer "B.Cu") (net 16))
 (segment (start 189.3 99.55) (end 189.3 95.65) (width 0.4) (layer "B.Cu") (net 14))
 (segment (start 189.35 95.65) (end 190 95) (width 0.4) (layer "B.Cu") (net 14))
 (segment (start 189.3 95.65) (end 189.35 95.65) (width 0.4) (layer "B.Cu") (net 14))
 (segment (start 203.7 84.3) (end 203.7 81.45) (width 0.4) (layer "B.Cu") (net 13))
 (segment (start 203 85) (end 203.7 84.3) (width 0.4) (layer "B.Cu") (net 13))
 (segment (start 203 95) (end 203.6 95.6) (width 0.4) (layer "B.Cu") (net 8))
 (segment (start 203.6 95.6) (end 203.6 99.55) (width 0.4) (layer "B.Cu") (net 8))
 (segment (start 192 95) (end 192 99.5) (width 0.4) (layer "B.Cu") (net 15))
 (segment (start 192 99.5) (end 191.9 99.6) (width 0.4) (layer "B.Cu") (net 15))
 (segment (start 198.25 84.55) (end 198.25 81.45) (width 0.4) (layer "B.Cu") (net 11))
 (segment (start 198.7 85) (end 198.25 84.55) (width 0.4) (layer "B.Cu") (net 11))
 (segment (start 201 85) (end 201 81.5) (width 0.4) (layer "B.Cu") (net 12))
 (segment (start 201 81.5) (end 200.95 81.45) (width 0.4) (layer "B.Cu") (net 12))
 (segment (start 198.3 95.7) (end 199 95) (width 0.4) (layer "B.Cu") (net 6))
 (segment (start 198.3 99.55) (end 198.3 95.7) (width 0.4) (layer "B.Cu") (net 6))
 (segment (start 200.95 99.6) (end 200.95 95.05) (width 0.4) (layer "B.Cu") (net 7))
 (segment (start 200.95 95.05) (end 201 95) (width 0.4) (layer "B.Cu") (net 7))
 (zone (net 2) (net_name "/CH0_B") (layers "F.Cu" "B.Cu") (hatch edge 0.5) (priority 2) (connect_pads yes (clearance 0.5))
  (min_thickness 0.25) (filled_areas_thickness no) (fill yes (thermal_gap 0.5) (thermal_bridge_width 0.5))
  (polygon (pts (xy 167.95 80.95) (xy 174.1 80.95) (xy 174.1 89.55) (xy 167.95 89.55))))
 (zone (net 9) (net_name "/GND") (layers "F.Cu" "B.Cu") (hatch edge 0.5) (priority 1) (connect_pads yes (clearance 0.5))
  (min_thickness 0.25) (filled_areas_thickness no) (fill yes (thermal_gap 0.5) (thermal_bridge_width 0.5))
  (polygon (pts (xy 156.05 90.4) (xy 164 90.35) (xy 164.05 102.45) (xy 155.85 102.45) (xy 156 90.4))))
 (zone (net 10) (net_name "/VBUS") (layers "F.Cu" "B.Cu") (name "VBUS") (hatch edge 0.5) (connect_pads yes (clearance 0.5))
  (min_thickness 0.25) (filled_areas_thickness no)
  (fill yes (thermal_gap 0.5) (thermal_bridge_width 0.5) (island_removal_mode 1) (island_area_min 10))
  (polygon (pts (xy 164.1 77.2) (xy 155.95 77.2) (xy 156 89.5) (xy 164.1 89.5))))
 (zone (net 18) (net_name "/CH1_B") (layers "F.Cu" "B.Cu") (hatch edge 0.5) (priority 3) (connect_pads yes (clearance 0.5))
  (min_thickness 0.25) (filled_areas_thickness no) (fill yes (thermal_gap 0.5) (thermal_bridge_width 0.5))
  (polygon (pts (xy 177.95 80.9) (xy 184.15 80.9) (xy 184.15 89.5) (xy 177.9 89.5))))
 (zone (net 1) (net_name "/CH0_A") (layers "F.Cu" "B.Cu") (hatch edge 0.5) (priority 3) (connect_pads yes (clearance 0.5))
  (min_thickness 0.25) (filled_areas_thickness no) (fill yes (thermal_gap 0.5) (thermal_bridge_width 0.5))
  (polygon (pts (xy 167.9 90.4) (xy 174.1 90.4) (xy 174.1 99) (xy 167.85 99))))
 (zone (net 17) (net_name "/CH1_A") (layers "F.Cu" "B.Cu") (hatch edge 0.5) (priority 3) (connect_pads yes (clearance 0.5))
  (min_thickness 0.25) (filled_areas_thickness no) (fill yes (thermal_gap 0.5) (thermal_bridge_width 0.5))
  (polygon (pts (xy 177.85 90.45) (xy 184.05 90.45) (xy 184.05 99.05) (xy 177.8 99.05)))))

